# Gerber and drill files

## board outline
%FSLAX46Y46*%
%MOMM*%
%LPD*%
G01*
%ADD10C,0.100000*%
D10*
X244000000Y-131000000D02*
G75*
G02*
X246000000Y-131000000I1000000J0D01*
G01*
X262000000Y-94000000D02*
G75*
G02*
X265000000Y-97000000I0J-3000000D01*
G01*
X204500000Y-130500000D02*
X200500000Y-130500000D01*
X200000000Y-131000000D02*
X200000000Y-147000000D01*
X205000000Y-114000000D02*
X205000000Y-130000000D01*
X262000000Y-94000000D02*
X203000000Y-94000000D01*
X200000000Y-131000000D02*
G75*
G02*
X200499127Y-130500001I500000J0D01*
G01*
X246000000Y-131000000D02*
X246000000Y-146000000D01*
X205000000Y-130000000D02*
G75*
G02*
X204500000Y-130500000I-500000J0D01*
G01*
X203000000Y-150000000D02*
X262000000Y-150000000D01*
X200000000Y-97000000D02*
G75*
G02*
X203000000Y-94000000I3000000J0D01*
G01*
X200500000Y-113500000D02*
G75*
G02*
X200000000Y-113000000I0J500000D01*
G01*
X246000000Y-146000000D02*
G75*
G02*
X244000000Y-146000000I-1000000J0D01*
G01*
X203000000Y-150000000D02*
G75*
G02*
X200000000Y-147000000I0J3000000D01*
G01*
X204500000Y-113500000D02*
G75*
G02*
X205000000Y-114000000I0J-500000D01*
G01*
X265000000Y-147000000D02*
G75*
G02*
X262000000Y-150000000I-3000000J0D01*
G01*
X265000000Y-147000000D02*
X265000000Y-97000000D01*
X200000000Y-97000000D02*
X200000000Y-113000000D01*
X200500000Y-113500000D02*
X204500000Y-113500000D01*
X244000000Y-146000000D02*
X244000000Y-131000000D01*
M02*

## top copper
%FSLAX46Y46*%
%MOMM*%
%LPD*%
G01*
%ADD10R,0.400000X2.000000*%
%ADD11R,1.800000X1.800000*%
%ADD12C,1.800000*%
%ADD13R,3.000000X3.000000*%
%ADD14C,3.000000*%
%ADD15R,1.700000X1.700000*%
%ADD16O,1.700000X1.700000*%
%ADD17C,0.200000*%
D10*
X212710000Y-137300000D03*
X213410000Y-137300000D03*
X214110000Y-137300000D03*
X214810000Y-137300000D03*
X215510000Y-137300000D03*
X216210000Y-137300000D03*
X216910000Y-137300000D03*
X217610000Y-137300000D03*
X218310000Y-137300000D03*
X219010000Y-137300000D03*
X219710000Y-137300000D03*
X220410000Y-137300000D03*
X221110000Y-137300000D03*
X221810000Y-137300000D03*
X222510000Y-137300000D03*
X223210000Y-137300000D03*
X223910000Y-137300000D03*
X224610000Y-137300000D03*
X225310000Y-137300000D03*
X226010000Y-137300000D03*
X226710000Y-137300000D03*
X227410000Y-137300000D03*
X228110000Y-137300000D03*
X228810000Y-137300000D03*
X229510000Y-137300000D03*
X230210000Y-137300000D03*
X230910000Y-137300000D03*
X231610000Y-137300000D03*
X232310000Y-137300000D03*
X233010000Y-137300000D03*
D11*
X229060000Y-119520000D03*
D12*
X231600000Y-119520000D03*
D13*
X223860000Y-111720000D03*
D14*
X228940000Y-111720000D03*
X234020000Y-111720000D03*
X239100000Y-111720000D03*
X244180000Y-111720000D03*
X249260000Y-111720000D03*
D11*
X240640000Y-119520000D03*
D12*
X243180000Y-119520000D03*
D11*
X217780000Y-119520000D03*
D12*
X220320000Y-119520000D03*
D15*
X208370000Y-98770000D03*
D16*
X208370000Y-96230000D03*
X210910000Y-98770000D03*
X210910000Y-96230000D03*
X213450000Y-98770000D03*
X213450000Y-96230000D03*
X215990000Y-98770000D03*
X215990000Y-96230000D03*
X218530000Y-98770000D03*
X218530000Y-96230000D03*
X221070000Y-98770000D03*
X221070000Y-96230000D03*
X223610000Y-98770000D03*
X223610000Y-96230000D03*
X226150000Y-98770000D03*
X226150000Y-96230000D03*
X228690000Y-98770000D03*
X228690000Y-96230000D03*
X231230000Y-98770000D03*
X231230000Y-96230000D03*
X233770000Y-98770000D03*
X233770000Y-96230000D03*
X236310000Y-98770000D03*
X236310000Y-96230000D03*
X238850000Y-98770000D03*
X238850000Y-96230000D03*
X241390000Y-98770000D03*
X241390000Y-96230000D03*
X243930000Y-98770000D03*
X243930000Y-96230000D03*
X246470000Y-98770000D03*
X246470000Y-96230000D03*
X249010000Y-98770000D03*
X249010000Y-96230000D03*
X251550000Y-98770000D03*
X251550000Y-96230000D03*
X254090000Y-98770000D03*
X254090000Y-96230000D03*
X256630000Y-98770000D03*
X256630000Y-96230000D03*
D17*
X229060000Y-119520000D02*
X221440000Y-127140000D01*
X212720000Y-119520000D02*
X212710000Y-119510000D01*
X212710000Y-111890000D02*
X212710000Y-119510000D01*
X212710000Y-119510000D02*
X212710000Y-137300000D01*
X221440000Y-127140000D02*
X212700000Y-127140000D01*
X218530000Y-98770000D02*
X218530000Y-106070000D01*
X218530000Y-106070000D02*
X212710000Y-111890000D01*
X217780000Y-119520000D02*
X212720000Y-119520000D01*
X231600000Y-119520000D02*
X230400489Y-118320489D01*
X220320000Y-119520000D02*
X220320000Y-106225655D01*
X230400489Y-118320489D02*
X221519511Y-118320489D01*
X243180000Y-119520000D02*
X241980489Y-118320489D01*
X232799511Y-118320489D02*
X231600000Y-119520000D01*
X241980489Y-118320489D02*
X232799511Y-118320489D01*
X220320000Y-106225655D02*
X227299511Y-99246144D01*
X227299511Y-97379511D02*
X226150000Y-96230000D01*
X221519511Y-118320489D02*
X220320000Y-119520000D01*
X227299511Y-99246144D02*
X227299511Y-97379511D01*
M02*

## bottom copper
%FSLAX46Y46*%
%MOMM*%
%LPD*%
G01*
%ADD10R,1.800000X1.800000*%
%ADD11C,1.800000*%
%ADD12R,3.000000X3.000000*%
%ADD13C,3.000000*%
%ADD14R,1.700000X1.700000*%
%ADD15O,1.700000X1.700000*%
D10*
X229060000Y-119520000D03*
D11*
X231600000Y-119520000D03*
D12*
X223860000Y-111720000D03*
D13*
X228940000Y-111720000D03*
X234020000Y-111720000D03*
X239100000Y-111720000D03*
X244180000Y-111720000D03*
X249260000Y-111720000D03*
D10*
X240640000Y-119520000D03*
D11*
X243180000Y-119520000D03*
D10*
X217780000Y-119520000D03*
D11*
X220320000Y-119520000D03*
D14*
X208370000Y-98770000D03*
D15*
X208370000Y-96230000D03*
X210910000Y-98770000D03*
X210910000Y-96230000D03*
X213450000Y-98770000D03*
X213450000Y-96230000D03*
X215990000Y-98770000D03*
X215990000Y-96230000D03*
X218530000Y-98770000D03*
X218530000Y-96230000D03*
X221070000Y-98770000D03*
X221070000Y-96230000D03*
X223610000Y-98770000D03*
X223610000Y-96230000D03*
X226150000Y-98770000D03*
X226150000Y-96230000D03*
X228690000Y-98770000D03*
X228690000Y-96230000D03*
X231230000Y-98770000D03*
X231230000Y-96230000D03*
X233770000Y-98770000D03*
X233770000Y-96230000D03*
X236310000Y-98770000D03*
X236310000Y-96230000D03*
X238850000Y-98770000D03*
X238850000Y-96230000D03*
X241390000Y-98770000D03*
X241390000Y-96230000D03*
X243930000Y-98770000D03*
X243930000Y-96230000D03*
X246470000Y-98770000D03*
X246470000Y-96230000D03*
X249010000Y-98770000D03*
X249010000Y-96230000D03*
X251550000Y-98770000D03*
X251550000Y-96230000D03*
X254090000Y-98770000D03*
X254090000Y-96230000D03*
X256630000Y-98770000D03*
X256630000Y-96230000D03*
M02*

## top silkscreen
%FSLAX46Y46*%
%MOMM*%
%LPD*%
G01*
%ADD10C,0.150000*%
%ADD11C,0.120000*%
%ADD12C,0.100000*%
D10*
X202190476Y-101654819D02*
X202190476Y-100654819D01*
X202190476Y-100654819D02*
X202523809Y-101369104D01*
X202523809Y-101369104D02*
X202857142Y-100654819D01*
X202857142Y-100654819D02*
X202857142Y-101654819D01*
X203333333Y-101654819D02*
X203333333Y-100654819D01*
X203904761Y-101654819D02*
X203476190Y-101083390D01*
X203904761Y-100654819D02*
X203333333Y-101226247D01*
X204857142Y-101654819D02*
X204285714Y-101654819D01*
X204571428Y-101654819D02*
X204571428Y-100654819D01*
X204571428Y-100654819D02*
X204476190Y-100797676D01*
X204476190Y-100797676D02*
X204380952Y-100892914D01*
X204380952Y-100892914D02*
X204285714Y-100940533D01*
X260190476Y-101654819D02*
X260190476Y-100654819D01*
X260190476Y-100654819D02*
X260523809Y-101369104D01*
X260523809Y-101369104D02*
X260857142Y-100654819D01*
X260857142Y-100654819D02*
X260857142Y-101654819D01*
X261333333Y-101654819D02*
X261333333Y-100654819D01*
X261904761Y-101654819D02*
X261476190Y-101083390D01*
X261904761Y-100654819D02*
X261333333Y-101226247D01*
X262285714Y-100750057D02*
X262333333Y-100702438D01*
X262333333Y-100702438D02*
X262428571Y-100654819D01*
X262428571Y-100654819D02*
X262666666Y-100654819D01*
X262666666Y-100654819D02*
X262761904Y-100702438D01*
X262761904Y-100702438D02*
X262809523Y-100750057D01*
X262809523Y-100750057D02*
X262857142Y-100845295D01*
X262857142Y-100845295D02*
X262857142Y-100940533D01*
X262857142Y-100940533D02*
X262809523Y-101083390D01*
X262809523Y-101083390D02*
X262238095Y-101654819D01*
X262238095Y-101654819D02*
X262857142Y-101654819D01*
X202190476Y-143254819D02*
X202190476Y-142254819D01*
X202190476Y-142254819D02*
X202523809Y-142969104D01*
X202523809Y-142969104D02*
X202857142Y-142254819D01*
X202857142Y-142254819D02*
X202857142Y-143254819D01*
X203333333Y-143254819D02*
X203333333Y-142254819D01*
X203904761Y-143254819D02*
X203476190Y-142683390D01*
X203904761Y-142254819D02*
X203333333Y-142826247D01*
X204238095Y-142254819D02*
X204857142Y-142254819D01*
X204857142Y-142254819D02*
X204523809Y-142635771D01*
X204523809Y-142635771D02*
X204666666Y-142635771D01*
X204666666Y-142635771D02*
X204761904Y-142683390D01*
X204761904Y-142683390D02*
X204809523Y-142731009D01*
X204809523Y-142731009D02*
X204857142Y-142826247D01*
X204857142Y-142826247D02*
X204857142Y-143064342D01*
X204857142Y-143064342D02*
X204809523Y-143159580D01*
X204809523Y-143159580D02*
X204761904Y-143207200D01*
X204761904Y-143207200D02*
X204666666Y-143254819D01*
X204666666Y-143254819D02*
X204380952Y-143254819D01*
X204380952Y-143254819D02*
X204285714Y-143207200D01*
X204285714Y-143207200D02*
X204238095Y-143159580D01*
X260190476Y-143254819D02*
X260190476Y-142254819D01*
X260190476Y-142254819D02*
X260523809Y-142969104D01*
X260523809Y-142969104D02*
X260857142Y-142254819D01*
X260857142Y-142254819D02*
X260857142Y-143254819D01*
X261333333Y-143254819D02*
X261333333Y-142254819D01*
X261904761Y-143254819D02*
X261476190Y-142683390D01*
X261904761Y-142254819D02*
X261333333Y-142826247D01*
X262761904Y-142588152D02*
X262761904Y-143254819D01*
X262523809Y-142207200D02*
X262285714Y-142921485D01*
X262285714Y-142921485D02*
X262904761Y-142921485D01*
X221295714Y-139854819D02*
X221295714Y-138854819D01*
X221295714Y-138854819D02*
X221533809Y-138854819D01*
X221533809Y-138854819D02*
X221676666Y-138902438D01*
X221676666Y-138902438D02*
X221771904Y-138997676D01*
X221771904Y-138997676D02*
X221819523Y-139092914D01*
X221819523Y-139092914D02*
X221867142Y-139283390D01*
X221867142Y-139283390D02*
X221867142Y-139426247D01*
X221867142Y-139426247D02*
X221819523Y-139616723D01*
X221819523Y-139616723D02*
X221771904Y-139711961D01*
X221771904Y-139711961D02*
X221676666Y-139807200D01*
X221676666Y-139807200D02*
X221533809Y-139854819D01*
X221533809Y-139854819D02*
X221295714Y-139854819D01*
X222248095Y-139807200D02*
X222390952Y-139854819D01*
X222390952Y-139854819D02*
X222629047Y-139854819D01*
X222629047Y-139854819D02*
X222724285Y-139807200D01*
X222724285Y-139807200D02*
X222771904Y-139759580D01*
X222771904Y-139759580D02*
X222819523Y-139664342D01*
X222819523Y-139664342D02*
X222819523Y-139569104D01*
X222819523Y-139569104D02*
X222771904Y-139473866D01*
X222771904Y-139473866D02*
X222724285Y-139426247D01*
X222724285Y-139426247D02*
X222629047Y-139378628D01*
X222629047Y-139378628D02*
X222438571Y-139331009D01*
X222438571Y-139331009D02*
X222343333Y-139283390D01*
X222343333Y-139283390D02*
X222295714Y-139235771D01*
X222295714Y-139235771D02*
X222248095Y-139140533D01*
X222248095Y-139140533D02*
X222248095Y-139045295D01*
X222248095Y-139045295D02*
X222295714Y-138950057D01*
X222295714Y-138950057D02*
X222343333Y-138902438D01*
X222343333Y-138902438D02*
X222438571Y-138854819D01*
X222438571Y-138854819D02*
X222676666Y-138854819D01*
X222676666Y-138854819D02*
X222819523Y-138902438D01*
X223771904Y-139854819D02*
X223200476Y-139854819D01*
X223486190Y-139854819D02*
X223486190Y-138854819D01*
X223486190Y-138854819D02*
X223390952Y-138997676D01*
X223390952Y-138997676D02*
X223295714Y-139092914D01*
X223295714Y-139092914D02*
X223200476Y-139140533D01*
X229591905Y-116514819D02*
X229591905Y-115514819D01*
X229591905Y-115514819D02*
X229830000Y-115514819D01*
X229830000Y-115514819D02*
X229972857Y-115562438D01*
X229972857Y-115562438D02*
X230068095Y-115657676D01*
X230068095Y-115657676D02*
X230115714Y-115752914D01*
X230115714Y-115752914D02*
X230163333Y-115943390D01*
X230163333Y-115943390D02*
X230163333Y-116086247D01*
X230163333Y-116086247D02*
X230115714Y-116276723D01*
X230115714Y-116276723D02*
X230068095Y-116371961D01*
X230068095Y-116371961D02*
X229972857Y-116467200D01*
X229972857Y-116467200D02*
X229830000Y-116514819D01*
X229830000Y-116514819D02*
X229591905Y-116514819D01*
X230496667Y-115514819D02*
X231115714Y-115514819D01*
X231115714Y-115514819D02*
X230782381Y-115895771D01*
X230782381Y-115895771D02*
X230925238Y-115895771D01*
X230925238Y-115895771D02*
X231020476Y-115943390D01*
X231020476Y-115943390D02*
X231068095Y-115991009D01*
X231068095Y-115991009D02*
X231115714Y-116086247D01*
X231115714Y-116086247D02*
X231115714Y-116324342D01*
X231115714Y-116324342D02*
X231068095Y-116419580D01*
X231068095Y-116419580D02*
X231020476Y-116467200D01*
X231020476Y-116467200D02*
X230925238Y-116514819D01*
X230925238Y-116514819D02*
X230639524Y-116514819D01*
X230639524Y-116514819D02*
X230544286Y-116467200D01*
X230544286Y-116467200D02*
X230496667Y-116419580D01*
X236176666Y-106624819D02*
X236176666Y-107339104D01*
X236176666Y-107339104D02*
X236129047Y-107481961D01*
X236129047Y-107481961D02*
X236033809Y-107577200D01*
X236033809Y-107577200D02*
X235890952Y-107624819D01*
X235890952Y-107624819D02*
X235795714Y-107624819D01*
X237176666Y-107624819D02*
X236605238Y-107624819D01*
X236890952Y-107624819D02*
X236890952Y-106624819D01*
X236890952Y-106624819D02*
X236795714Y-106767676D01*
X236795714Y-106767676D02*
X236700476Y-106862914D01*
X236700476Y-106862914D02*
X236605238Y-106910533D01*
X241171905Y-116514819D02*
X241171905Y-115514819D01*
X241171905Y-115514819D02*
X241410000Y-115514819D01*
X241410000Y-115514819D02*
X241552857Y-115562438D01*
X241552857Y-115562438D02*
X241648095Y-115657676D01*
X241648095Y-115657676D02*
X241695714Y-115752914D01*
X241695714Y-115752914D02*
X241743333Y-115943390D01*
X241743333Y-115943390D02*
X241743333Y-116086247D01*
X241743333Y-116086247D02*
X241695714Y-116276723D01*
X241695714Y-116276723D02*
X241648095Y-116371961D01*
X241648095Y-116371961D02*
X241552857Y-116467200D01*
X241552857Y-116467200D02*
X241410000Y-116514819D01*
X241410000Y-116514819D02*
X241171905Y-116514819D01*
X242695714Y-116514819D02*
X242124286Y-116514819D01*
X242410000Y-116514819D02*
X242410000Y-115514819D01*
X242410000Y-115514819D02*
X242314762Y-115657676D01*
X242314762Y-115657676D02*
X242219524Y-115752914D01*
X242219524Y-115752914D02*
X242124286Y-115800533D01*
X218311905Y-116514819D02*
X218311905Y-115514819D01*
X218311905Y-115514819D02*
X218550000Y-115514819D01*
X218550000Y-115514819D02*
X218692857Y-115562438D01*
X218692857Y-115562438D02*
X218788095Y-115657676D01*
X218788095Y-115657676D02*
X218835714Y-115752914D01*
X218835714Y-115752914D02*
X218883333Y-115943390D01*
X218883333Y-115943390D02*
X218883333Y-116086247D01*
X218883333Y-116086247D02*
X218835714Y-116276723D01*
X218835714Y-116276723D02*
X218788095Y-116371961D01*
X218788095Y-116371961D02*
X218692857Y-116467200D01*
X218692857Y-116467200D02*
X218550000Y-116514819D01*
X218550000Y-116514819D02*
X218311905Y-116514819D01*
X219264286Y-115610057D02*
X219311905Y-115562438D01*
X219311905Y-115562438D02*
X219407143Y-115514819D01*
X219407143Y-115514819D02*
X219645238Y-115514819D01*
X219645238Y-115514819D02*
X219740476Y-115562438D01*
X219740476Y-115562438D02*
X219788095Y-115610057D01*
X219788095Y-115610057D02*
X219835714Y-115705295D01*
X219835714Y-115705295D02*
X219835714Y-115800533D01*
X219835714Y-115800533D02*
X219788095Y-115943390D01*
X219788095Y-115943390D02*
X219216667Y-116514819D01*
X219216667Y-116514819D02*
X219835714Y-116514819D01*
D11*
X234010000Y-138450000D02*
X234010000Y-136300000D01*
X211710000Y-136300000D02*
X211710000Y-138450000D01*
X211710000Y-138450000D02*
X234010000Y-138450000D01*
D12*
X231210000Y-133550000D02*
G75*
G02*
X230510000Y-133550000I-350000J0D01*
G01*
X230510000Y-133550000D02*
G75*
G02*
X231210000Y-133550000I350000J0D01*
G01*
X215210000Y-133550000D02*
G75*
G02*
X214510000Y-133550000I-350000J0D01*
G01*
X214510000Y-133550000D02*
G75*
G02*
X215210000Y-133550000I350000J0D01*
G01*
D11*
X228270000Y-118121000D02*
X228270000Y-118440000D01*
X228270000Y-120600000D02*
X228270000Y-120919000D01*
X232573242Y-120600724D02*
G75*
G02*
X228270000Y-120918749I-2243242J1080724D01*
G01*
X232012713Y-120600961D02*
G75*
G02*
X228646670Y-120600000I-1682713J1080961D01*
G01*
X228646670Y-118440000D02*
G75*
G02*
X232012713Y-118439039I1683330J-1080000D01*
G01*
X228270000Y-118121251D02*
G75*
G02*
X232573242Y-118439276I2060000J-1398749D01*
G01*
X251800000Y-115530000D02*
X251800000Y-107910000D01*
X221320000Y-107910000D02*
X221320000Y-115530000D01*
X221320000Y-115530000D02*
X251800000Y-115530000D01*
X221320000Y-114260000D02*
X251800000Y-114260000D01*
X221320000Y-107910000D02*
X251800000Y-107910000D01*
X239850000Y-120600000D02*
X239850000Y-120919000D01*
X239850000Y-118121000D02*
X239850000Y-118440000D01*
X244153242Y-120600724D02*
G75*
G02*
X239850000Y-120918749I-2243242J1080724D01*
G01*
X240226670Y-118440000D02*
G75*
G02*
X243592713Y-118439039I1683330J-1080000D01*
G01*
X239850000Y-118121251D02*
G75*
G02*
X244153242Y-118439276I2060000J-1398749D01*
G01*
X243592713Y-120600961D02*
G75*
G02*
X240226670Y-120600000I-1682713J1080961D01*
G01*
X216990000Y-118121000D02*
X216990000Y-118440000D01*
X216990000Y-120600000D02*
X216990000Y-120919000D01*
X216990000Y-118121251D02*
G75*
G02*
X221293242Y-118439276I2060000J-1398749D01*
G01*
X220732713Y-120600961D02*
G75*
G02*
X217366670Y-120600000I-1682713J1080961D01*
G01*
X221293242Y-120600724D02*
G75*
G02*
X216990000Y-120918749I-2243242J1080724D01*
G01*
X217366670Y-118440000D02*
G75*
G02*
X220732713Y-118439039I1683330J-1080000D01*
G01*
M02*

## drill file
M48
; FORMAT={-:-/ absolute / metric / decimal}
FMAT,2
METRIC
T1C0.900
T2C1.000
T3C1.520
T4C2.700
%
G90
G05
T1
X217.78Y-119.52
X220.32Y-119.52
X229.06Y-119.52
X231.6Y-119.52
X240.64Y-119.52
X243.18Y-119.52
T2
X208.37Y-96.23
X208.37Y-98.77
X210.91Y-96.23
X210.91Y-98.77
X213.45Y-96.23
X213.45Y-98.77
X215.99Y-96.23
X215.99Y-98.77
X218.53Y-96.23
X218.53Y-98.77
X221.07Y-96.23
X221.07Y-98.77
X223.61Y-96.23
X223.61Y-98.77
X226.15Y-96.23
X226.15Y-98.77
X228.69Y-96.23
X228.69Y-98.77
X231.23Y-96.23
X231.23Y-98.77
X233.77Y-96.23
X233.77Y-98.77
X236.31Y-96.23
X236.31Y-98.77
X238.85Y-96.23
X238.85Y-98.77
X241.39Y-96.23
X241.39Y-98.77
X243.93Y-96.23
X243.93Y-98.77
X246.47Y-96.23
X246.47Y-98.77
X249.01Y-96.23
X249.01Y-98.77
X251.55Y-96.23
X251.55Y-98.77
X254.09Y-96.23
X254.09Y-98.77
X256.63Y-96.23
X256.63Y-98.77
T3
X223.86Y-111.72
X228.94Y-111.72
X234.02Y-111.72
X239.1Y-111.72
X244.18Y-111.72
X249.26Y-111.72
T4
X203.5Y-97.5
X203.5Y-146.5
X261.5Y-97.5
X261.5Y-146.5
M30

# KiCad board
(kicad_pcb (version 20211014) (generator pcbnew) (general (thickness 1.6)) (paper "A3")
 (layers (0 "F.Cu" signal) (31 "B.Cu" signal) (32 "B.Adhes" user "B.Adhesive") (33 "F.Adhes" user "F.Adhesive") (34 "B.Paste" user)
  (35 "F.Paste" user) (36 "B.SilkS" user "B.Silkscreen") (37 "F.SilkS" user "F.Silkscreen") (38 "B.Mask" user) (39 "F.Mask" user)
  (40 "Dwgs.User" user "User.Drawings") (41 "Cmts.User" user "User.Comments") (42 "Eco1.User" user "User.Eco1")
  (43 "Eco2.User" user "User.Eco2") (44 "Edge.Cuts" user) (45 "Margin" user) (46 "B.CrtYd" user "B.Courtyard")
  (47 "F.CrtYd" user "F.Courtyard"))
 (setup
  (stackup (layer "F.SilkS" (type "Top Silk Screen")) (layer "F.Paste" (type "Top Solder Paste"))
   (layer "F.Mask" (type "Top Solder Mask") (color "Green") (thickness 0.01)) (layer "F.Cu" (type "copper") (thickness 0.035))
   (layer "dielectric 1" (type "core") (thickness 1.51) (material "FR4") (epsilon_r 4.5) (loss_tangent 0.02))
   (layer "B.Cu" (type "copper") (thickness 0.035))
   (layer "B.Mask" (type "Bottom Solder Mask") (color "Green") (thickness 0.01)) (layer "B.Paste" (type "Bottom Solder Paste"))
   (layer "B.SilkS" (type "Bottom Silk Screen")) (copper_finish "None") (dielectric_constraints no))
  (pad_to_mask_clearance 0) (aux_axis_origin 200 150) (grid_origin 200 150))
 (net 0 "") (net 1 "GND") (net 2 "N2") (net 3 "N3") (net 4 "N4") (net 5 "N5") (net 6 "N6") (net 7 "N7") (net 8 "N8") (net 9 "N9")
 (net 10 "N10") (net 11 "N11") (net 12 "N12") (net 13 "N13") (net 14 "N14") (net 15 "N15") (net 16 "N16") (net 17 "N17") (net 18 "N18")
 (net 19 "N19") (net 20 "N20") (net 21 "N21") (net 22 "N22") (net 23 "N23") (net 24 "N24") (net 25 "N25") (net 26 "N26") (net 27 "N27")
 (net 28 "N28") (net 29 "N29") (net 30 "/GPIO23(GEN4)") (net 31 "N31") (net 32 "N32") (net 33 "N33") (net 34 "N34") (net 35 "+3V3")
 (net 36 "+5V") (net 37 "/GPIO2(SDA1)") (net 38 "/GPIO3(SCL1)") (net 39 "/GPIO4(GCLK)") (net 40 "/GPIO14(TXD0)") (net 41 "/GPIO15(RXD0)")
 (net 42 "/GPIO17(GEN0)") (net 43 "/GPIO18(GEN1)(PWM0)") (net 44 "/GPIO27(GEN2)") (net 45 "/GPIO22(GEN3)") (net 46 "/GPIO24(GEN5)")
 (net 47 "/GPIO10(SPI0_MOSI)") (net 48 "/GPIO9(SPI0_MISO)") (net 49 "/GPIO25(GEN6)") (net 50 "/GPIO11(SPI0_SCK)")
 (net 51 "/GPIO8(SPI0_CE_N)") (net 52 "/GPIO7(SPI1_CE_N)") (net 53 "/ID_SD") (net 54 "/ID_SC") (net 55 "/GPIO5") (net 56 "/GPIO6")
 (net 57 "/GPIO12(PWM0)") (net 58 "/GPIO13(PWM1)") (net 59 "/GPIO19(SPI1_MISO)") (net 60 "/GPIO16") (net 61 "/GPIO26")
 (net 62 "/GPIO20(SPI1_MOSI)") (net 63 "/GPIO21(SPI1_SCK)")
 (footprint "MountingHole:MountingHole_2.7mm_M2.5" (layer "F.Cu") (at 203.5 97.5 180)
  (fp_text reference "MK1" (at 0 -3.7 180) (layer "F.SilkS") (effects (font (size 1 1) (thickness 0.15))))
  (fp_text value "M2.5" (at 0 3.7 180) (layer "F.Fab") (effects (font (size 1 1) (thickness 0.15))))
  (pad "" np_thru_hole circle locked (at 0 0 180) (size 2.7 2.7) (drill 2.7) (layers *.Cu *.Mask)))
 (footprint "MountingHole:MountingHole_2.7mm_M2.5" (layer "F.Cu") (at 261.5 97.5 180)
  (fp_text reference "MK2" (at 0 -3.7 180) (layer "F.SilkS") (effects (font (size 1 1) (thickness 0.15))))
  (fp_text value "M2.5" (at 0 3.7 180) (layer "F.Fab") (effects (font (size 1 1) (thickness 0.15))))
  (pad "" np_thru_hole circle locked (at 0 0 180) (size 2.7 2.7) (drill 2.7) (layers *.Cu *.Mask)))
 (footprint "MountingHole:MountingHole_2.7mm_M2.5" (layer "F.Cu") (at 203.5 146.5)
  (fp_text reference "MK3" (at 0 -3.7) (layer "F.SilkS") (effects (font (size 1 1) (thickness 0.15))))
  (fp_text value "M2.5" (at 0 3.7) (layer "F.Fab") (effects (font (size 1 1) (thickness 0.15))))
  (pad "" np_thru_hole circle locked (at 0 0) (size 2.7 2.7) (drill 2.7) (layers *.Cu *.Mask)))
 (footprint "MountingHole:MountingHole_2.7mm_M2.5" (layer "F.Cu") (at 261.5 146.5)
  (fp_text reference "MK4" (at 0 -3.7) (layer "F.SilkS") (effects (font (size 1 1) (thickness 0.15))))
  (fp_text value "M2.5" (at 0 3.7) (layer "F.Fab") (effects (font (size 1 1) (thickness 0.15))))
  (pad "" np_thru_hole circle locked (at 0 0) (size 2.7 2.7) (drill 2.7) (layers *.Cu *.Mask)))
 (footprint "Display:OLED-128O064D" (layer "F.Cu") (at 222.86 137.3)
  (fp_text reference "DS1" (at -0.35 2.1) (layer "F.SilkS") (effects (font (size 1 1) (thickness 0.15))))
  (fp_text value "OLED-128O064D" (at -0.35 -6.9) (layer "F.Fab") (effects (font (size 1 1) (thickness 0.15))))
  (fp_line (start 11.15 1.15) (end 11.15 -1) (layer "F.SilkS") (width 0.12))
  (fp_line (start -11.15 -1) (end -11.15 1.15) (layer "F.SilkS") (width 0.12))
  (fp_line (start -11.15 1.15) (end 11.15 1.15) (layer "F.SilkS") (width 0.12))
  (fp_circle (center 8 -3.75) (end 8.35 -3.75) (layer "F.SilkS") (width 0.1) (fill none))
  (fp_circle (center -8 -3.75) (end -7.65 -3.75) (layer "F.SilkS") (width 0.1) (fill none))
  (pad "1" smd rect (at -10.15 0) (size 0.4 2) (layers "F.Cu" "F.Paste" "F.Mask") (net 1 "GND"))
  (pad "2" smd rect (at -9.45 0) (size 0.4 2) (layers "F.Cu" "F.Paste" "F.Mask") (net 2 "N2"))
  (pad "3" smd rect (at -8.75 0) (size 0.4 2) (layers "F.Cu" "F.Paste" "F.Mask") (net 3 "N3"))
  (pad "4" smd rect (at -8.05 0) (size 0.4 2) (layers "F.Cu" "F.Paste" "F.Mask") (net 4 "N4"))
  (pad "5" smd rect (at -7.35 0) (size 0.4 2) (layers "F.Cu" "F.Paste" "F.Mask") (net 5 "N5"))
  (pad "6" smd rect (at -6.65 0) (size 0.4 2) (layers "F.Cu" "F.Paste" "F.Mask") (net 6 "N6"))
  (pad "7" smd rect (at -5.95 0) (size 0.4 2) (layers "F.Cu" "F.Paste" "F.Mask") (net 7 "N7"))
  (pad "8" smd rect (at -5.25 0) (size 0.4 2) (layers "F.Cu" "F.Paste" "F.Mask") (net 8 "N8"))
  (pad "9" smd rect (at -4.55 0) (size 0.4 2) (layers "F.Cu" "F.Paste" "F.Mask") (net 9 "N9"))
  (pad "10" smd rect (at -3.85 0) (size 0.4 2) (layers "F.Cu" "F.Paste" "F.Mask") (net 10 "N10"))
  (pad "11" smd rect (at -3.15 0) (size 0.4 2) (layers "F.Cu" "F.Paste" "F.Mask") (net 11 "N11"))
  (pad "12" smd rect (at -2.45 0) (size 0.4 2) (layers "F.Cu" "F.Paste" "F.Mask") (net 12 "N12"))
  (pad "13" smd rect (at -1.75 0) (size 0.4 2) (layers "F.Cu" "F.Paste" "F.Mask") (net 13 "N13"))
  (pad "14" smd rect (at -1.05 0) (size 0.4 2) (layers "F.Cu" "F.Paste" "F.Mask") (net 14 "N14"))
  (pad "15" smd rect (at -0.35 0) (size 0.4 2) (layers "F.Cu" "F.Paste" "F.Mask") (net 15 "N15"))
  (pad "16" smd rect (at 0.35 0) (size 0.4 2) (layers "F.Cu" "F.Paste" "F.Mask") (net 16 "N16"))
  (pad "17" smd rect (at 1.05 0) (size 0.4 2) (layers "F.Cu" "F.Paste" "F.Mask") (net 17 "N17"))
  (pad "18" smd rect (at 1.75 0) (size 0.4 2) (layers "F.Cu" "F.Paste" "F.Mask") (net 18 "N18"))
  (pad "19" smd rect (at 2.45 0) (size 0.4 2) (layers "F.Cu" "F.Paste" "F.Mask") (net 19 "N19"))
  (pad "20" smd rect (at 3.15 0) (size 0.4 2) (layers "F.Cu" "F.Paste" "F.Mask") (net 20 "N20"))
  (pad "21" smd rect (at 3.85 0) (size 0.4 2) (layers "F.Cu" "F.Paste" "F.Mask") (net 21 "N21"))
  (pad "22" smd rect (at 4.55 0) (size 0.4 2) (layers "F.Cu" "F.Paste" "F.Mask") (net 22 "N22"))
  (pad "23" smd rect (at 5.25 0) (size 0.4 2) (layers "F.Cu" "F.Paste" "F.Mask") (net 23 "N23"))
  (pad "24" smd rect (at 5.95 0) (size 0.4 2) (layers "F.Cu" "F.Paste" "F.Mask") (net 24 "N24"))
  (pad "25" smd rect (at 6.65 0) (size 0.4 2) (layers "F.Cu" "F.Paste" "F.Mask") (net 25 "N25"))
  (pad "26" smd rect (at 7.35 0) (size 0.4 2) (layers "F.Cu" "F.Paste" "F.Mask") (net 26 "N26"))
  (pad "27" smd rect (at 8.05 0) (size 0.4 2) (layers "F.Cu" "F.Paste" "F.Mask") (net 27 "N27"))
  (pad "28" smd rect (at 8.75 0) (size 0.4 2) (layers "F.Cu" "F.Paste" "F.Mask") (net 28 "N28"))
  (pad "29" smd rect (at 9.45 0) (size 0.4 2) (layers "F.Cu" "F.Paste" "F.Mask") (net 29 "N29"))
  (pad "30" smd rect (at 10.15 0) (size 0.4 2) (layers "F.Cu" "F.Paste" "F.Mask") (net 1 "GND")))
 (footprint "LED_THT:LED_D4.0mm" (layer "F.Cu") (at 229.06 119.52)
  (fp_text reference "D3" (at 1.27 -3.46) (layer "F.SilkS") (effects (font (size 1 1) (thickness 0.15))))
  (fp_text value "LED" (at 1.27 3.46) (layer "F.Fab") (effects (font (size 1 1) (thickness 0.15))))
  (fp_line (start -0.79 -1.399) (end -0.79 -1.08) (layer "F.SilkS") (width 0.12))
  (fp_line (start -0.79 1.08) (end -0.79 1.399) (layer "F.SilkS") (width 0.12))
  (fp_arc (start 3.513242 1.080724) (mid 1.453519 2.483228) (end -0.79 1.398749) (layer "F.SilkS") (width 0.12))
  (fp_arc (start 2.952713 1.080961) (mid 1.269429 2) (end -0.41333 1.08) (layer "F.SilkS") (width 0.12))
  (fp_arc (start -0.41333 -1.08) (mid 1.269429 -2) (end 2.952713 -1.080961) (layer "F.SilkS") (width 0.12))
  (fp_arc (start -0.79 -1.398749) (mid 1.453519 -2.483228) (end 3.513242 -1.080724) (layer "F.SilkS") (width 0.12))
  (pad "1" thru_hole rect (at 0 0) (size 1.8 1.8) (drill 0.9) (layers *.Cu *.Mask) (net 1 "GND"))
  (pad "2" thru_hole circle (at 2.54 0) (size 1.8 1.8) (drill 0.9) (layers *.Cu *.Mask) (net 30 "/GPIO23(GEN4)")))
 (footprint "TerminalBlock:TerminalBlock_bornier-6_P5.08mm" (layer "F.Cu") (at 223.86 111.72)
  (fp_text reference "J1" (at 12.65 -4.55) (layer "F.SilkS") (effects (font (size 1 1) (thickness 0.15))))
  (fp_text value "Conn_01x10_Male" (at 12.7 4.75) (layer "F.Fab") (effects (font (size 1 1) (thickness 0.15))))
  (fp_line (start 27.94 3.81) (end 27.94 -3.81) (layer "F.SilkS") (width 0.12))
  (fp_line (start -2.54 -3.81) (end -2.54 3.81) (layer "F.SilkS") (width 0.12))
  (fp_line (start -2.54 3.81) (end 27.94 3.81) (layer "F.SilkS") (width 0.12))
  (fp_line (start -2.54 2.54) (end 27.94 2.54) (layer "F.SilkS") (width 0.12))
  (fp_line (start -2.54 -3.81) (end 27.94 -3.81) (layer "F.SilkS") (width 0.12))
  (pad "1" thru_hole rect (at 0 0) (size 3 3) (drill 1.52) (layers *.Cu *.Mask) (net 8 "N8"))
  (pad "2" thru_hole circle (at 5.08 0) (size 3 3) (drill 1.52) (layers *.Cu *.Mask) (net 29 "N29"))
  (pad "3" thru_hole circle (at 10.16 0) (size 3 3) (drill 1.52) (layers *.Cu *.Mask) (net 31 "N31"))
  (pad "4" thru_hole circle (at 15.24 0) (size 3 3) (drill 1.52) (layers *.Cu *.Mask) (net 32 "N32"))
  (pad "5" thru_hole circle (at 20.32 0) (size 3 3) (drill 1.52) (layers *.Cu *.Mask) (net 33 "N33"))
  (pad "6" thru_hole circle (at 25.4 0) (size 3 3) (drill 1.52) (layers *.Cu *.Mask) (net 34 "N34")))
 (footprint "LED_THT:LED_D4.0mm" (layer "F.Cu") (at 240.64 119.52)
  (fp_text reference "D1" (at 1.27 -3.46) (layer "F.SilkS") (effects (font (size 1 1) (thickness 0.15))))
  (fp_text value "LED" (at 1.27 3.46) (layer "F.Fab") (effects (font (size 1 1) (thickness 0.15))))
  (fp_line (start -0.79 1.08) (end -0.79 1.399) (layer "F.SilkS") (width 0.12))
  (fp_line (start -0.79 -1.399) (end -0.79 -1.08) (layer "F.SilkS") (width 0.12))
  (fp_arc (start 3.513242 1.080724) (mid 1.453519 2.483228) (end -0.79 1.398749) (layer "F.SilkS") (width 0.12))
  (fp_arc (start -0.41333 -1.08) (mid 1.269429 -2) (end 2.952713 -1.080961) (layer "F.SilkS") (width 0.12))
  (fp_arc (start -0.79 -1.398749) (mid 1.453519 -2.483228) (end 3.513242 -1.080724) (layer "F.SilkS") (width 0.12))
  (fp_arc (start 2.952713 1.080961) (mid 1.269429 2) (end -0.41333 1.08) (layer "F.SilkS") (width 0.12))
  (pad "1" thru_hole rect (at 0 0) (size 1.8 1.8) (drill 0.9) (layers *.Cu *.Mask) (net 1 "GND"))
  (pad "2" thru_hole circle (at 2.54 0) (size 1.8 1.8) (drill 0.9) (layers *.Cu *.Mask) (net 30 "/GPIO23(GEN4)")))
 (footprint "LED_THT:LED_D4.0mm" (layer "F.Cu") (at 217.78 119.52)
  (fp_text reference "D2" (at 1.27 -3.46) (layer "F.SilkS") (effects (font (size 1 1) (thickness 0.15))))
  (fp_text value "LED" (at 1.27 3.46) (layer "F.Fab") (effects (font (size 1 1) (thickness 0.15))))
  (fp_line (start -0.79 -1.399) (end -0.79 -1.08) (layer "F.SilkS") (width 0.12))
  (fp_line (start -0.79 1.08) (end -0.79 1.399) (layer "F.SilkS") (width 0.12))
  (fp_arc (start -0.79 -1.398749) (mid 1.453519 -2.483228) (end 3.513242 -1.080724) (layer "F.SilkS") (width 0.12))
  (fp_arc (start 2.952713 1.080961) (mid 1.269429 2) (end -0.41333 1.08) (layer "F.SilkS") (width 0.12))
  (fp_arc (start 3.513242 1.080724) (mid 1.453519 2.483228) (end -0.79 1.398749) (layer "F.SilkS") (width 0.12))
  (fp_arc (start -0.41333 -1.08) (mid 1.269429 -2) (end 2.952713 -1.080961) (layer "F.SilkS") (width 0.12))
  (pad "1" thru_hole rect (at 0 0) (size 1.8 1.8) (drill 0.9) (layers *.Cu *.Mask) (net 1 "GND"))
  (pad "2" thru_hole circle (at 2.54 0) (size 1.8 1.8) (drill 0.9) (layers *.Cu *.Mask) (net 30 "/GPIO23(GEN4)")))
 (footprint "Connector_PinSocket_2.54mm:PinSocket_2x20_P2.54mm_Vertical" (layer "B.Cu") (at 208.37 98.77 -90)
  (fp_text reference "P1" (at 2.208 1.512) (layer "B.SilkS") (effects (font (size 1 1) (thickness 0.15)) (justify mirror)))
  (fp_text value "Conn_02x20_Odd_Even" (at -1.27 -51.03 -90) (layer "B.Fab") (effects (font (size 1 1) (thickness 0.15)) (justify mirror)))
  (pad "1" thru_hole rect locked (at 0 0 270) (size 1.7 1.7) (drill 1) (layers *.Cu *.Mask) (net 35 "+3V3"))
  (pad "2" thru_hole oval locked (at -2.54 0 270) (size 1.7 1.7) (drill 1) (layers *.Cu *.Mask) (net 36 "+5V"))
  (pad "3" thru_hole oval locked (at 0 -2.54 270) (size 1.7 1.7) (drill 1) (layers *.Cu *.Mask) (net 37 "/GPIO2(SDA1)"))
  (pad "4" thru_hole oval locked (at -2.54 -2.54 270) (size 1.7 1.7) (drill 1) (layers *.Cu *.Mask) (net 36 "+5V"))
  (pad "5" thru_hole oval locked (at 0 -5.08 270) (size 1.7 1.7) (drill 1) (layers *.Cu *.Mask) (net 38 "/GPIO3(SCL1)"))
  (pad "6" thru_hole oval locked (at -2.54 -5.08 270) (size 1.7 1.7) (drill 1) (layers *.Cu *.Mask) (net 1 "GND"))
  (pad "7" thru_hole oval locked (at 0 -7.62 270) (size 1.7 1.7) (drill 1) (layers *.Cu *.Mask) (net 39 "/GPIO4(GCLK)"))
  (pad "8" thru_hole oval locked (at -2.54 -7.62 270) (size 1.7 1.7) (drill 1) (layers *.Cu *.Mask) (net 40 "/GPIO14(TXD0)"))
  (pad "9" thru_hole oval locked (at 0 -10.16 270) (size 1.7 1.7) (drill 1) (layers *.Cu *.Mask) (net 1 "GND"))
  (pad "10" thru_hole oval locked (at -2.54 -10.16 270) (size 1.7 1.7) (drill 1) (layers *.Cu *.Mask) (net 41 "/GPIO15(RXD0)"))
  (pad "11" thru_hole oval locked (at 0 -12.7 270) (size 1.7 1.7) (drill 1) (layers *.Cu *.Mask) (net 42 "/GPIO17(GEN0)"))
  (pad "12" thru_hole oval locked (at -2.54 -12.7 270) (size 1.7 1.7) (drill 1) (layers *.Cu *.Mask) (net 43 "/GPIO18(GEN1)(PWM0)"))
  (pad "13" thru_hole oval locked (at 0 -15.24 270) (size 1.7 1.7) (drill 1) (layers *.Cu *.Mask) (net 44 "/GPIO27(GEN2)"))
  (pad "14" thru_hole oval locked (at -2.54 -15.24 270) (size 1.7 1.7) (drill 1) (layers *.Cu *.Mask) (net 1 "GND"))
  (pad "15" thru_hole oval locked (at 0 -17.78 270) (size 1.7 1.7) (drill 1) (layers *.Cu *.Mask) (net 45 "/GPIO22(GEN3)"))
  (pad "16" thru_hole oval locked (at -2.54 -17.78 270) (size 1.7 1.7) (drill 1) (layers *.Cu *.Mask) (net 30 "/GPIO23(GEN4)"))
  (pad "17" thru_hole oval locked (at 0 -20.32 270) (size 1.7 1.7) (drill 1) (layers *.Cu *.Mask) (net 35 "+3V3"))
  (pad "18" thru_hole oval locked (at -2.54 -20.32 270) (size 1.7 1.7) (drill 1) (layers *.Cu *.Mask) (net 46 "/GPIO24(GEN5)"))
  (pad "19" thru_hole oval locked (at 0 -22.86 270) (size 1.7 1.7) (drill 1) (layers *.Cu *.Mask) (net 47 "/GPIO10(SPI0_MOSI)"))
  (pad "20" thru_hole oval locked (at -2.54 -22.86 270) (size 1.7 1.7) (drill 1) (layers *.Cu *.Mask) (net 1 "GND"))
  (pad "21" thru_hole oval locked (at 0 -25.4 270) (size 1.7 1.7) (drill 1) (layers *.Cu *.Mask) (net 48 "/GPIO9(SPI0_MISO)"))
  (pad "22" thru_hole oval locked (at -2.54 -25.4 270) (size 1.7 1.7) (drill 1) (layers *.Cu *.Mask) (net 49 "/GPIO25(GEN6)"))
  (pad "23" thru_hole oval locked (at 0 -27.94 270) (size 1.7 1.7) (drill 1) (layers *.Cu *.Mask) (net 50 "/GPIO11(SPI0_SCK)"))
  (pad "24" thru_hole oval locked (at -2.54 -27.94 270) (size 1.7 1.7) (drill 1) (layers *.Cu *.Mask) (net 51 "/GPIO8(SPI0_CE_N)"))
  (pad "25" thru_hole oval locked (at 0 -30.48 270) (size 1.7 1.7) (drill 1) (layers *.Cu *.Mask) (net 1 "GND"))
  (pad "26" thru_hole oval locked (at -2.54 -30.48 270) (size 1.7 1.7) (drill 1) (layers *.Cu *.Mask) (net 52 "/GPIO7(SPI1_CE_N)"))
  (pad "27" thru_hole oval locked (at 0 -33.02 270) (size 1.7 1.7) (drill 1) (layers *.Cu *.Mask) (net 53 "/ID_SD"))
  (pad "28" thru_hole oval locked (at -2.54 -33.02 270) (size 1.7 1.7) (drill 1) (layers *.Cu *.Mask) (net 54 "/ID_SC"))
  (pad "29" thru_hole oval locked (at 0 -35.56 270) (size 1.7 1.7) (drill 1) (layers *.Cu *.Mask) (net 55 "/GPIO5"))
  (pad "30" thru_hole oval locked (at -2.54 -35.56 270) (size 1.7 1.7) (drill 1) (layers *.Cu *.Mask) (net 1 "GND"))
  (pad "31" thru_hole oval locked (at 0 -38.1 270) (size 1.7 1.7) (drill 1) (layers *.Cu *.Mask) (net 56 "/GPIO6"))
  (pad "32" thru_hole oval locked (at -2.54 -38.1 270) (size 1.7 1.7) (drill 1) (layers *.Cu *.Mask) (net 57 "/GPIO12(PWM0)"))
  (pad "33" thru_hole oval locked (at 0 -40.64 270) (size 1.7 1.7) (drill 1) (layers *.Cu *.Mask) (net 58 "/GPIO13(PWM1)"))
  (pad "34" thru_hole oval locked (at -2.54 -40.64 270) (size 1.7 1.7) (drill 1) (layers *.Cu *.Mask) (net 1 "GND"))
  (pad "35" thru_hole oval locked (at 0 -43.18 270) (size 1.7 1.7) (drill 1) (layers *.Cu *.Mask) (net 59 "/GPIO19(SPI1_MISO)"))
  (pad "36" thru_hole oval locked (at -2.54 -43.18 270) (size 1.7 1.7) (drill 1) (layers *.Cu *.Mask) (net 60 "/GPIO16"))
  (pad "37" thru_hole oval locked (at 0 -45.72 270) (size 1.7 1.7) (drill 1) (layers *.Cu *.Mask) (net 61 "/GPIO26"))
  (pad "38" thru_hole oval locked (at -2.54 -45.72 270) (size 1.7 1.7) (drill 1) (layers *.Cu *.Mask) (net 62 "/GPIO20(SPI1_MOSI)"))
  (pad "39" thru_hole oval locked (at 0 -48.26 270) (size 1.7 1.7) (drill 1) (layers *.Cu *.Mask) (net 1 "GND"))
  (pad "40" thru_hole oval locked (at -2.54 -48.26 270) (size 1.7 1.7) (drill 1) (layers *.Cu *.Mask) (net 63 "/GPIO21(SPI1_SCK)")))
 (gr_arc (start 244 131) (mid 245 130) (end 246 131) (layer "Edge.Cuts") (width 0.1))
 (gr_arc (start 262 94) (mid 264.12132 94.87868) (end 265 97) (layer "Edge.Cuts") (width 0.1))
 (gr_line (start 204.5 130.5) (end 200.5 130.5) (layer "Edge.Cuts") (width 0.1))
 (gr_line (start 200 131) (end 200 147) (layer "Edge.Cuts") (width 0.1))
 (gr_line (start 205 114) (end 205 130) (layer "Edge.Cuts") (width 0.1))
 (gr_line (start 262 94) (end 203 94) (layer "Edge.Cuts") (width 0.1))
 (gr_arc (start 200 131) (mid 200.146138 130.646755) (end 200.499127 130.500001) (layer "Edge.Cuts") (width 0.1))
 (gr_line (start 246 131) (end 246 146) (layer "Edge.Cuts") (width 0.1))
 (gr_arc (start 205 130) (mid 204.853553 130.353553) (end 204.5 130.5) (layer "Edge.Cuts") (width 0.1))
 (gr_line (start 203 150) (end 262 150) (layer "Edge.Cuts") (width 0.1))
 (gr_arc (start 200 97) (mid 200.87868 94.87868) (end 203 94) (layer "Edge.Cuts") (width 0.1))
 (gr_arc (start 200.5 113.5) (mid 200.146447 113.353553) (end 200 113) (layer "Edge.Cuts") (width 0.1))
 (gr_arc (start 246 146) (mid 245 147) (end 244 146) (layer "Edge.Cuts") (width 0.1))
 (gr_arc (start 203 150) (mid 200.87868 149.12132) (end 200 147) (layer "Edge.Cuts") (width 0.1))
 (gr_arc (start 204.5 113.5) (mid 204.853553 113.646447) (end 205 114) (layer "Edge.Cuts") (width 0.1))
 (gr_arc (start 265 147) (mid 264.12132 149.12132) (end 262 150) (layer "Edge.Cuts") (width 0.1))
 (gr_line (start 265 147) (end 265 97) (layer "Edge.Cuts") (width 0.1))
 (gr_line (start 200 97) (end 200 113) (layer "Edge.Cuts") (width 0.1))
 (gr_line (start 200.5 113.5) (end 204.5 113.5) (layer "Edge.Cuts") (width 0.1))
 (gr_line (start 244 146) (end 244 131) (layer "Edge.Cuts") (width 0.1))
 (segment (start 229.06 119.52) (end 221.44 127.14) (width 0.2) (layer "F.Cu") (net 1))
 (segment (start 212.72 119.52) (end 212.71 119.51) (width 0.2) (layer "F.Cu") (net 1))
 (segment (start 212.71 111.89) (end 212.71 119.51) (width 0.2) (layer "F.Cu") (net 1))
 (segment (start 212.71 119.51) (end 212.71 137.3) (width 0.2) (layer "F.Cu") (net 1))
 (segment (start 221.44 127.14) (end 212.7 127.14) (width 0.2) (layer "F.Cu") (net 1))
 (segment (start 218.53 98.77) (end 218.53 106.07) (width 0.2) (layer "F.Cu") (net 1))
 (segment (start 218.53 106.07) (end 212.71 111.89) (width 0.2) (layer "F.Cu") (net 1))
 (segment (start 217.78 119.52) (end 212.72 119.52) (width 0.2) (layer "F.Cu") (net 1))
 (segment (start 231.6 119.52) (end 230.400489 118.320489) (width 0.2) (layer "F.Cu") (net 30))
 (segment (start 220.32 119.52) (end 220.32 106.225655) (width 0.2) (layer "F.Cu") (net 30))
 (segment (start 230.400489 118.320489) (end 221.519511 118.320489) (width 0.2) (layer "F.Cu") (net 30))
 (segment (start 243.18 119.52) (end 241.980489 118.320489) (width 0.2) (layer "F.Cu") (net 30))
 (segment (start 232.799511 118.320489) (end 231.6 119.52) (width 0.2) (layer "F.Cu") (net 30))
 (segment (start 241.980489 118.320489) (end 232.799511 118.320489) (width 0.2) (layer "F.Cu") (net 30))
 (segment (start 220.32 106.225655) (end 227.299511 99.246144) (width 0.2) (layer "F.Cu") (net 30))
 (segment (start 227.299511 97.379511) (end 226.15 96.23) (width 0.2) (layer "F.Cu") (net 30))
 (segment (start 221.519511 118.320489) (end 220.32 119.52) (width 0.2) (layer "F.Cu") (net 30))
 (segment (start 227.299511 99.246144) (end 227.299511 97.379511) (width 0.2) (layer "F.Cu") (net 30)))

